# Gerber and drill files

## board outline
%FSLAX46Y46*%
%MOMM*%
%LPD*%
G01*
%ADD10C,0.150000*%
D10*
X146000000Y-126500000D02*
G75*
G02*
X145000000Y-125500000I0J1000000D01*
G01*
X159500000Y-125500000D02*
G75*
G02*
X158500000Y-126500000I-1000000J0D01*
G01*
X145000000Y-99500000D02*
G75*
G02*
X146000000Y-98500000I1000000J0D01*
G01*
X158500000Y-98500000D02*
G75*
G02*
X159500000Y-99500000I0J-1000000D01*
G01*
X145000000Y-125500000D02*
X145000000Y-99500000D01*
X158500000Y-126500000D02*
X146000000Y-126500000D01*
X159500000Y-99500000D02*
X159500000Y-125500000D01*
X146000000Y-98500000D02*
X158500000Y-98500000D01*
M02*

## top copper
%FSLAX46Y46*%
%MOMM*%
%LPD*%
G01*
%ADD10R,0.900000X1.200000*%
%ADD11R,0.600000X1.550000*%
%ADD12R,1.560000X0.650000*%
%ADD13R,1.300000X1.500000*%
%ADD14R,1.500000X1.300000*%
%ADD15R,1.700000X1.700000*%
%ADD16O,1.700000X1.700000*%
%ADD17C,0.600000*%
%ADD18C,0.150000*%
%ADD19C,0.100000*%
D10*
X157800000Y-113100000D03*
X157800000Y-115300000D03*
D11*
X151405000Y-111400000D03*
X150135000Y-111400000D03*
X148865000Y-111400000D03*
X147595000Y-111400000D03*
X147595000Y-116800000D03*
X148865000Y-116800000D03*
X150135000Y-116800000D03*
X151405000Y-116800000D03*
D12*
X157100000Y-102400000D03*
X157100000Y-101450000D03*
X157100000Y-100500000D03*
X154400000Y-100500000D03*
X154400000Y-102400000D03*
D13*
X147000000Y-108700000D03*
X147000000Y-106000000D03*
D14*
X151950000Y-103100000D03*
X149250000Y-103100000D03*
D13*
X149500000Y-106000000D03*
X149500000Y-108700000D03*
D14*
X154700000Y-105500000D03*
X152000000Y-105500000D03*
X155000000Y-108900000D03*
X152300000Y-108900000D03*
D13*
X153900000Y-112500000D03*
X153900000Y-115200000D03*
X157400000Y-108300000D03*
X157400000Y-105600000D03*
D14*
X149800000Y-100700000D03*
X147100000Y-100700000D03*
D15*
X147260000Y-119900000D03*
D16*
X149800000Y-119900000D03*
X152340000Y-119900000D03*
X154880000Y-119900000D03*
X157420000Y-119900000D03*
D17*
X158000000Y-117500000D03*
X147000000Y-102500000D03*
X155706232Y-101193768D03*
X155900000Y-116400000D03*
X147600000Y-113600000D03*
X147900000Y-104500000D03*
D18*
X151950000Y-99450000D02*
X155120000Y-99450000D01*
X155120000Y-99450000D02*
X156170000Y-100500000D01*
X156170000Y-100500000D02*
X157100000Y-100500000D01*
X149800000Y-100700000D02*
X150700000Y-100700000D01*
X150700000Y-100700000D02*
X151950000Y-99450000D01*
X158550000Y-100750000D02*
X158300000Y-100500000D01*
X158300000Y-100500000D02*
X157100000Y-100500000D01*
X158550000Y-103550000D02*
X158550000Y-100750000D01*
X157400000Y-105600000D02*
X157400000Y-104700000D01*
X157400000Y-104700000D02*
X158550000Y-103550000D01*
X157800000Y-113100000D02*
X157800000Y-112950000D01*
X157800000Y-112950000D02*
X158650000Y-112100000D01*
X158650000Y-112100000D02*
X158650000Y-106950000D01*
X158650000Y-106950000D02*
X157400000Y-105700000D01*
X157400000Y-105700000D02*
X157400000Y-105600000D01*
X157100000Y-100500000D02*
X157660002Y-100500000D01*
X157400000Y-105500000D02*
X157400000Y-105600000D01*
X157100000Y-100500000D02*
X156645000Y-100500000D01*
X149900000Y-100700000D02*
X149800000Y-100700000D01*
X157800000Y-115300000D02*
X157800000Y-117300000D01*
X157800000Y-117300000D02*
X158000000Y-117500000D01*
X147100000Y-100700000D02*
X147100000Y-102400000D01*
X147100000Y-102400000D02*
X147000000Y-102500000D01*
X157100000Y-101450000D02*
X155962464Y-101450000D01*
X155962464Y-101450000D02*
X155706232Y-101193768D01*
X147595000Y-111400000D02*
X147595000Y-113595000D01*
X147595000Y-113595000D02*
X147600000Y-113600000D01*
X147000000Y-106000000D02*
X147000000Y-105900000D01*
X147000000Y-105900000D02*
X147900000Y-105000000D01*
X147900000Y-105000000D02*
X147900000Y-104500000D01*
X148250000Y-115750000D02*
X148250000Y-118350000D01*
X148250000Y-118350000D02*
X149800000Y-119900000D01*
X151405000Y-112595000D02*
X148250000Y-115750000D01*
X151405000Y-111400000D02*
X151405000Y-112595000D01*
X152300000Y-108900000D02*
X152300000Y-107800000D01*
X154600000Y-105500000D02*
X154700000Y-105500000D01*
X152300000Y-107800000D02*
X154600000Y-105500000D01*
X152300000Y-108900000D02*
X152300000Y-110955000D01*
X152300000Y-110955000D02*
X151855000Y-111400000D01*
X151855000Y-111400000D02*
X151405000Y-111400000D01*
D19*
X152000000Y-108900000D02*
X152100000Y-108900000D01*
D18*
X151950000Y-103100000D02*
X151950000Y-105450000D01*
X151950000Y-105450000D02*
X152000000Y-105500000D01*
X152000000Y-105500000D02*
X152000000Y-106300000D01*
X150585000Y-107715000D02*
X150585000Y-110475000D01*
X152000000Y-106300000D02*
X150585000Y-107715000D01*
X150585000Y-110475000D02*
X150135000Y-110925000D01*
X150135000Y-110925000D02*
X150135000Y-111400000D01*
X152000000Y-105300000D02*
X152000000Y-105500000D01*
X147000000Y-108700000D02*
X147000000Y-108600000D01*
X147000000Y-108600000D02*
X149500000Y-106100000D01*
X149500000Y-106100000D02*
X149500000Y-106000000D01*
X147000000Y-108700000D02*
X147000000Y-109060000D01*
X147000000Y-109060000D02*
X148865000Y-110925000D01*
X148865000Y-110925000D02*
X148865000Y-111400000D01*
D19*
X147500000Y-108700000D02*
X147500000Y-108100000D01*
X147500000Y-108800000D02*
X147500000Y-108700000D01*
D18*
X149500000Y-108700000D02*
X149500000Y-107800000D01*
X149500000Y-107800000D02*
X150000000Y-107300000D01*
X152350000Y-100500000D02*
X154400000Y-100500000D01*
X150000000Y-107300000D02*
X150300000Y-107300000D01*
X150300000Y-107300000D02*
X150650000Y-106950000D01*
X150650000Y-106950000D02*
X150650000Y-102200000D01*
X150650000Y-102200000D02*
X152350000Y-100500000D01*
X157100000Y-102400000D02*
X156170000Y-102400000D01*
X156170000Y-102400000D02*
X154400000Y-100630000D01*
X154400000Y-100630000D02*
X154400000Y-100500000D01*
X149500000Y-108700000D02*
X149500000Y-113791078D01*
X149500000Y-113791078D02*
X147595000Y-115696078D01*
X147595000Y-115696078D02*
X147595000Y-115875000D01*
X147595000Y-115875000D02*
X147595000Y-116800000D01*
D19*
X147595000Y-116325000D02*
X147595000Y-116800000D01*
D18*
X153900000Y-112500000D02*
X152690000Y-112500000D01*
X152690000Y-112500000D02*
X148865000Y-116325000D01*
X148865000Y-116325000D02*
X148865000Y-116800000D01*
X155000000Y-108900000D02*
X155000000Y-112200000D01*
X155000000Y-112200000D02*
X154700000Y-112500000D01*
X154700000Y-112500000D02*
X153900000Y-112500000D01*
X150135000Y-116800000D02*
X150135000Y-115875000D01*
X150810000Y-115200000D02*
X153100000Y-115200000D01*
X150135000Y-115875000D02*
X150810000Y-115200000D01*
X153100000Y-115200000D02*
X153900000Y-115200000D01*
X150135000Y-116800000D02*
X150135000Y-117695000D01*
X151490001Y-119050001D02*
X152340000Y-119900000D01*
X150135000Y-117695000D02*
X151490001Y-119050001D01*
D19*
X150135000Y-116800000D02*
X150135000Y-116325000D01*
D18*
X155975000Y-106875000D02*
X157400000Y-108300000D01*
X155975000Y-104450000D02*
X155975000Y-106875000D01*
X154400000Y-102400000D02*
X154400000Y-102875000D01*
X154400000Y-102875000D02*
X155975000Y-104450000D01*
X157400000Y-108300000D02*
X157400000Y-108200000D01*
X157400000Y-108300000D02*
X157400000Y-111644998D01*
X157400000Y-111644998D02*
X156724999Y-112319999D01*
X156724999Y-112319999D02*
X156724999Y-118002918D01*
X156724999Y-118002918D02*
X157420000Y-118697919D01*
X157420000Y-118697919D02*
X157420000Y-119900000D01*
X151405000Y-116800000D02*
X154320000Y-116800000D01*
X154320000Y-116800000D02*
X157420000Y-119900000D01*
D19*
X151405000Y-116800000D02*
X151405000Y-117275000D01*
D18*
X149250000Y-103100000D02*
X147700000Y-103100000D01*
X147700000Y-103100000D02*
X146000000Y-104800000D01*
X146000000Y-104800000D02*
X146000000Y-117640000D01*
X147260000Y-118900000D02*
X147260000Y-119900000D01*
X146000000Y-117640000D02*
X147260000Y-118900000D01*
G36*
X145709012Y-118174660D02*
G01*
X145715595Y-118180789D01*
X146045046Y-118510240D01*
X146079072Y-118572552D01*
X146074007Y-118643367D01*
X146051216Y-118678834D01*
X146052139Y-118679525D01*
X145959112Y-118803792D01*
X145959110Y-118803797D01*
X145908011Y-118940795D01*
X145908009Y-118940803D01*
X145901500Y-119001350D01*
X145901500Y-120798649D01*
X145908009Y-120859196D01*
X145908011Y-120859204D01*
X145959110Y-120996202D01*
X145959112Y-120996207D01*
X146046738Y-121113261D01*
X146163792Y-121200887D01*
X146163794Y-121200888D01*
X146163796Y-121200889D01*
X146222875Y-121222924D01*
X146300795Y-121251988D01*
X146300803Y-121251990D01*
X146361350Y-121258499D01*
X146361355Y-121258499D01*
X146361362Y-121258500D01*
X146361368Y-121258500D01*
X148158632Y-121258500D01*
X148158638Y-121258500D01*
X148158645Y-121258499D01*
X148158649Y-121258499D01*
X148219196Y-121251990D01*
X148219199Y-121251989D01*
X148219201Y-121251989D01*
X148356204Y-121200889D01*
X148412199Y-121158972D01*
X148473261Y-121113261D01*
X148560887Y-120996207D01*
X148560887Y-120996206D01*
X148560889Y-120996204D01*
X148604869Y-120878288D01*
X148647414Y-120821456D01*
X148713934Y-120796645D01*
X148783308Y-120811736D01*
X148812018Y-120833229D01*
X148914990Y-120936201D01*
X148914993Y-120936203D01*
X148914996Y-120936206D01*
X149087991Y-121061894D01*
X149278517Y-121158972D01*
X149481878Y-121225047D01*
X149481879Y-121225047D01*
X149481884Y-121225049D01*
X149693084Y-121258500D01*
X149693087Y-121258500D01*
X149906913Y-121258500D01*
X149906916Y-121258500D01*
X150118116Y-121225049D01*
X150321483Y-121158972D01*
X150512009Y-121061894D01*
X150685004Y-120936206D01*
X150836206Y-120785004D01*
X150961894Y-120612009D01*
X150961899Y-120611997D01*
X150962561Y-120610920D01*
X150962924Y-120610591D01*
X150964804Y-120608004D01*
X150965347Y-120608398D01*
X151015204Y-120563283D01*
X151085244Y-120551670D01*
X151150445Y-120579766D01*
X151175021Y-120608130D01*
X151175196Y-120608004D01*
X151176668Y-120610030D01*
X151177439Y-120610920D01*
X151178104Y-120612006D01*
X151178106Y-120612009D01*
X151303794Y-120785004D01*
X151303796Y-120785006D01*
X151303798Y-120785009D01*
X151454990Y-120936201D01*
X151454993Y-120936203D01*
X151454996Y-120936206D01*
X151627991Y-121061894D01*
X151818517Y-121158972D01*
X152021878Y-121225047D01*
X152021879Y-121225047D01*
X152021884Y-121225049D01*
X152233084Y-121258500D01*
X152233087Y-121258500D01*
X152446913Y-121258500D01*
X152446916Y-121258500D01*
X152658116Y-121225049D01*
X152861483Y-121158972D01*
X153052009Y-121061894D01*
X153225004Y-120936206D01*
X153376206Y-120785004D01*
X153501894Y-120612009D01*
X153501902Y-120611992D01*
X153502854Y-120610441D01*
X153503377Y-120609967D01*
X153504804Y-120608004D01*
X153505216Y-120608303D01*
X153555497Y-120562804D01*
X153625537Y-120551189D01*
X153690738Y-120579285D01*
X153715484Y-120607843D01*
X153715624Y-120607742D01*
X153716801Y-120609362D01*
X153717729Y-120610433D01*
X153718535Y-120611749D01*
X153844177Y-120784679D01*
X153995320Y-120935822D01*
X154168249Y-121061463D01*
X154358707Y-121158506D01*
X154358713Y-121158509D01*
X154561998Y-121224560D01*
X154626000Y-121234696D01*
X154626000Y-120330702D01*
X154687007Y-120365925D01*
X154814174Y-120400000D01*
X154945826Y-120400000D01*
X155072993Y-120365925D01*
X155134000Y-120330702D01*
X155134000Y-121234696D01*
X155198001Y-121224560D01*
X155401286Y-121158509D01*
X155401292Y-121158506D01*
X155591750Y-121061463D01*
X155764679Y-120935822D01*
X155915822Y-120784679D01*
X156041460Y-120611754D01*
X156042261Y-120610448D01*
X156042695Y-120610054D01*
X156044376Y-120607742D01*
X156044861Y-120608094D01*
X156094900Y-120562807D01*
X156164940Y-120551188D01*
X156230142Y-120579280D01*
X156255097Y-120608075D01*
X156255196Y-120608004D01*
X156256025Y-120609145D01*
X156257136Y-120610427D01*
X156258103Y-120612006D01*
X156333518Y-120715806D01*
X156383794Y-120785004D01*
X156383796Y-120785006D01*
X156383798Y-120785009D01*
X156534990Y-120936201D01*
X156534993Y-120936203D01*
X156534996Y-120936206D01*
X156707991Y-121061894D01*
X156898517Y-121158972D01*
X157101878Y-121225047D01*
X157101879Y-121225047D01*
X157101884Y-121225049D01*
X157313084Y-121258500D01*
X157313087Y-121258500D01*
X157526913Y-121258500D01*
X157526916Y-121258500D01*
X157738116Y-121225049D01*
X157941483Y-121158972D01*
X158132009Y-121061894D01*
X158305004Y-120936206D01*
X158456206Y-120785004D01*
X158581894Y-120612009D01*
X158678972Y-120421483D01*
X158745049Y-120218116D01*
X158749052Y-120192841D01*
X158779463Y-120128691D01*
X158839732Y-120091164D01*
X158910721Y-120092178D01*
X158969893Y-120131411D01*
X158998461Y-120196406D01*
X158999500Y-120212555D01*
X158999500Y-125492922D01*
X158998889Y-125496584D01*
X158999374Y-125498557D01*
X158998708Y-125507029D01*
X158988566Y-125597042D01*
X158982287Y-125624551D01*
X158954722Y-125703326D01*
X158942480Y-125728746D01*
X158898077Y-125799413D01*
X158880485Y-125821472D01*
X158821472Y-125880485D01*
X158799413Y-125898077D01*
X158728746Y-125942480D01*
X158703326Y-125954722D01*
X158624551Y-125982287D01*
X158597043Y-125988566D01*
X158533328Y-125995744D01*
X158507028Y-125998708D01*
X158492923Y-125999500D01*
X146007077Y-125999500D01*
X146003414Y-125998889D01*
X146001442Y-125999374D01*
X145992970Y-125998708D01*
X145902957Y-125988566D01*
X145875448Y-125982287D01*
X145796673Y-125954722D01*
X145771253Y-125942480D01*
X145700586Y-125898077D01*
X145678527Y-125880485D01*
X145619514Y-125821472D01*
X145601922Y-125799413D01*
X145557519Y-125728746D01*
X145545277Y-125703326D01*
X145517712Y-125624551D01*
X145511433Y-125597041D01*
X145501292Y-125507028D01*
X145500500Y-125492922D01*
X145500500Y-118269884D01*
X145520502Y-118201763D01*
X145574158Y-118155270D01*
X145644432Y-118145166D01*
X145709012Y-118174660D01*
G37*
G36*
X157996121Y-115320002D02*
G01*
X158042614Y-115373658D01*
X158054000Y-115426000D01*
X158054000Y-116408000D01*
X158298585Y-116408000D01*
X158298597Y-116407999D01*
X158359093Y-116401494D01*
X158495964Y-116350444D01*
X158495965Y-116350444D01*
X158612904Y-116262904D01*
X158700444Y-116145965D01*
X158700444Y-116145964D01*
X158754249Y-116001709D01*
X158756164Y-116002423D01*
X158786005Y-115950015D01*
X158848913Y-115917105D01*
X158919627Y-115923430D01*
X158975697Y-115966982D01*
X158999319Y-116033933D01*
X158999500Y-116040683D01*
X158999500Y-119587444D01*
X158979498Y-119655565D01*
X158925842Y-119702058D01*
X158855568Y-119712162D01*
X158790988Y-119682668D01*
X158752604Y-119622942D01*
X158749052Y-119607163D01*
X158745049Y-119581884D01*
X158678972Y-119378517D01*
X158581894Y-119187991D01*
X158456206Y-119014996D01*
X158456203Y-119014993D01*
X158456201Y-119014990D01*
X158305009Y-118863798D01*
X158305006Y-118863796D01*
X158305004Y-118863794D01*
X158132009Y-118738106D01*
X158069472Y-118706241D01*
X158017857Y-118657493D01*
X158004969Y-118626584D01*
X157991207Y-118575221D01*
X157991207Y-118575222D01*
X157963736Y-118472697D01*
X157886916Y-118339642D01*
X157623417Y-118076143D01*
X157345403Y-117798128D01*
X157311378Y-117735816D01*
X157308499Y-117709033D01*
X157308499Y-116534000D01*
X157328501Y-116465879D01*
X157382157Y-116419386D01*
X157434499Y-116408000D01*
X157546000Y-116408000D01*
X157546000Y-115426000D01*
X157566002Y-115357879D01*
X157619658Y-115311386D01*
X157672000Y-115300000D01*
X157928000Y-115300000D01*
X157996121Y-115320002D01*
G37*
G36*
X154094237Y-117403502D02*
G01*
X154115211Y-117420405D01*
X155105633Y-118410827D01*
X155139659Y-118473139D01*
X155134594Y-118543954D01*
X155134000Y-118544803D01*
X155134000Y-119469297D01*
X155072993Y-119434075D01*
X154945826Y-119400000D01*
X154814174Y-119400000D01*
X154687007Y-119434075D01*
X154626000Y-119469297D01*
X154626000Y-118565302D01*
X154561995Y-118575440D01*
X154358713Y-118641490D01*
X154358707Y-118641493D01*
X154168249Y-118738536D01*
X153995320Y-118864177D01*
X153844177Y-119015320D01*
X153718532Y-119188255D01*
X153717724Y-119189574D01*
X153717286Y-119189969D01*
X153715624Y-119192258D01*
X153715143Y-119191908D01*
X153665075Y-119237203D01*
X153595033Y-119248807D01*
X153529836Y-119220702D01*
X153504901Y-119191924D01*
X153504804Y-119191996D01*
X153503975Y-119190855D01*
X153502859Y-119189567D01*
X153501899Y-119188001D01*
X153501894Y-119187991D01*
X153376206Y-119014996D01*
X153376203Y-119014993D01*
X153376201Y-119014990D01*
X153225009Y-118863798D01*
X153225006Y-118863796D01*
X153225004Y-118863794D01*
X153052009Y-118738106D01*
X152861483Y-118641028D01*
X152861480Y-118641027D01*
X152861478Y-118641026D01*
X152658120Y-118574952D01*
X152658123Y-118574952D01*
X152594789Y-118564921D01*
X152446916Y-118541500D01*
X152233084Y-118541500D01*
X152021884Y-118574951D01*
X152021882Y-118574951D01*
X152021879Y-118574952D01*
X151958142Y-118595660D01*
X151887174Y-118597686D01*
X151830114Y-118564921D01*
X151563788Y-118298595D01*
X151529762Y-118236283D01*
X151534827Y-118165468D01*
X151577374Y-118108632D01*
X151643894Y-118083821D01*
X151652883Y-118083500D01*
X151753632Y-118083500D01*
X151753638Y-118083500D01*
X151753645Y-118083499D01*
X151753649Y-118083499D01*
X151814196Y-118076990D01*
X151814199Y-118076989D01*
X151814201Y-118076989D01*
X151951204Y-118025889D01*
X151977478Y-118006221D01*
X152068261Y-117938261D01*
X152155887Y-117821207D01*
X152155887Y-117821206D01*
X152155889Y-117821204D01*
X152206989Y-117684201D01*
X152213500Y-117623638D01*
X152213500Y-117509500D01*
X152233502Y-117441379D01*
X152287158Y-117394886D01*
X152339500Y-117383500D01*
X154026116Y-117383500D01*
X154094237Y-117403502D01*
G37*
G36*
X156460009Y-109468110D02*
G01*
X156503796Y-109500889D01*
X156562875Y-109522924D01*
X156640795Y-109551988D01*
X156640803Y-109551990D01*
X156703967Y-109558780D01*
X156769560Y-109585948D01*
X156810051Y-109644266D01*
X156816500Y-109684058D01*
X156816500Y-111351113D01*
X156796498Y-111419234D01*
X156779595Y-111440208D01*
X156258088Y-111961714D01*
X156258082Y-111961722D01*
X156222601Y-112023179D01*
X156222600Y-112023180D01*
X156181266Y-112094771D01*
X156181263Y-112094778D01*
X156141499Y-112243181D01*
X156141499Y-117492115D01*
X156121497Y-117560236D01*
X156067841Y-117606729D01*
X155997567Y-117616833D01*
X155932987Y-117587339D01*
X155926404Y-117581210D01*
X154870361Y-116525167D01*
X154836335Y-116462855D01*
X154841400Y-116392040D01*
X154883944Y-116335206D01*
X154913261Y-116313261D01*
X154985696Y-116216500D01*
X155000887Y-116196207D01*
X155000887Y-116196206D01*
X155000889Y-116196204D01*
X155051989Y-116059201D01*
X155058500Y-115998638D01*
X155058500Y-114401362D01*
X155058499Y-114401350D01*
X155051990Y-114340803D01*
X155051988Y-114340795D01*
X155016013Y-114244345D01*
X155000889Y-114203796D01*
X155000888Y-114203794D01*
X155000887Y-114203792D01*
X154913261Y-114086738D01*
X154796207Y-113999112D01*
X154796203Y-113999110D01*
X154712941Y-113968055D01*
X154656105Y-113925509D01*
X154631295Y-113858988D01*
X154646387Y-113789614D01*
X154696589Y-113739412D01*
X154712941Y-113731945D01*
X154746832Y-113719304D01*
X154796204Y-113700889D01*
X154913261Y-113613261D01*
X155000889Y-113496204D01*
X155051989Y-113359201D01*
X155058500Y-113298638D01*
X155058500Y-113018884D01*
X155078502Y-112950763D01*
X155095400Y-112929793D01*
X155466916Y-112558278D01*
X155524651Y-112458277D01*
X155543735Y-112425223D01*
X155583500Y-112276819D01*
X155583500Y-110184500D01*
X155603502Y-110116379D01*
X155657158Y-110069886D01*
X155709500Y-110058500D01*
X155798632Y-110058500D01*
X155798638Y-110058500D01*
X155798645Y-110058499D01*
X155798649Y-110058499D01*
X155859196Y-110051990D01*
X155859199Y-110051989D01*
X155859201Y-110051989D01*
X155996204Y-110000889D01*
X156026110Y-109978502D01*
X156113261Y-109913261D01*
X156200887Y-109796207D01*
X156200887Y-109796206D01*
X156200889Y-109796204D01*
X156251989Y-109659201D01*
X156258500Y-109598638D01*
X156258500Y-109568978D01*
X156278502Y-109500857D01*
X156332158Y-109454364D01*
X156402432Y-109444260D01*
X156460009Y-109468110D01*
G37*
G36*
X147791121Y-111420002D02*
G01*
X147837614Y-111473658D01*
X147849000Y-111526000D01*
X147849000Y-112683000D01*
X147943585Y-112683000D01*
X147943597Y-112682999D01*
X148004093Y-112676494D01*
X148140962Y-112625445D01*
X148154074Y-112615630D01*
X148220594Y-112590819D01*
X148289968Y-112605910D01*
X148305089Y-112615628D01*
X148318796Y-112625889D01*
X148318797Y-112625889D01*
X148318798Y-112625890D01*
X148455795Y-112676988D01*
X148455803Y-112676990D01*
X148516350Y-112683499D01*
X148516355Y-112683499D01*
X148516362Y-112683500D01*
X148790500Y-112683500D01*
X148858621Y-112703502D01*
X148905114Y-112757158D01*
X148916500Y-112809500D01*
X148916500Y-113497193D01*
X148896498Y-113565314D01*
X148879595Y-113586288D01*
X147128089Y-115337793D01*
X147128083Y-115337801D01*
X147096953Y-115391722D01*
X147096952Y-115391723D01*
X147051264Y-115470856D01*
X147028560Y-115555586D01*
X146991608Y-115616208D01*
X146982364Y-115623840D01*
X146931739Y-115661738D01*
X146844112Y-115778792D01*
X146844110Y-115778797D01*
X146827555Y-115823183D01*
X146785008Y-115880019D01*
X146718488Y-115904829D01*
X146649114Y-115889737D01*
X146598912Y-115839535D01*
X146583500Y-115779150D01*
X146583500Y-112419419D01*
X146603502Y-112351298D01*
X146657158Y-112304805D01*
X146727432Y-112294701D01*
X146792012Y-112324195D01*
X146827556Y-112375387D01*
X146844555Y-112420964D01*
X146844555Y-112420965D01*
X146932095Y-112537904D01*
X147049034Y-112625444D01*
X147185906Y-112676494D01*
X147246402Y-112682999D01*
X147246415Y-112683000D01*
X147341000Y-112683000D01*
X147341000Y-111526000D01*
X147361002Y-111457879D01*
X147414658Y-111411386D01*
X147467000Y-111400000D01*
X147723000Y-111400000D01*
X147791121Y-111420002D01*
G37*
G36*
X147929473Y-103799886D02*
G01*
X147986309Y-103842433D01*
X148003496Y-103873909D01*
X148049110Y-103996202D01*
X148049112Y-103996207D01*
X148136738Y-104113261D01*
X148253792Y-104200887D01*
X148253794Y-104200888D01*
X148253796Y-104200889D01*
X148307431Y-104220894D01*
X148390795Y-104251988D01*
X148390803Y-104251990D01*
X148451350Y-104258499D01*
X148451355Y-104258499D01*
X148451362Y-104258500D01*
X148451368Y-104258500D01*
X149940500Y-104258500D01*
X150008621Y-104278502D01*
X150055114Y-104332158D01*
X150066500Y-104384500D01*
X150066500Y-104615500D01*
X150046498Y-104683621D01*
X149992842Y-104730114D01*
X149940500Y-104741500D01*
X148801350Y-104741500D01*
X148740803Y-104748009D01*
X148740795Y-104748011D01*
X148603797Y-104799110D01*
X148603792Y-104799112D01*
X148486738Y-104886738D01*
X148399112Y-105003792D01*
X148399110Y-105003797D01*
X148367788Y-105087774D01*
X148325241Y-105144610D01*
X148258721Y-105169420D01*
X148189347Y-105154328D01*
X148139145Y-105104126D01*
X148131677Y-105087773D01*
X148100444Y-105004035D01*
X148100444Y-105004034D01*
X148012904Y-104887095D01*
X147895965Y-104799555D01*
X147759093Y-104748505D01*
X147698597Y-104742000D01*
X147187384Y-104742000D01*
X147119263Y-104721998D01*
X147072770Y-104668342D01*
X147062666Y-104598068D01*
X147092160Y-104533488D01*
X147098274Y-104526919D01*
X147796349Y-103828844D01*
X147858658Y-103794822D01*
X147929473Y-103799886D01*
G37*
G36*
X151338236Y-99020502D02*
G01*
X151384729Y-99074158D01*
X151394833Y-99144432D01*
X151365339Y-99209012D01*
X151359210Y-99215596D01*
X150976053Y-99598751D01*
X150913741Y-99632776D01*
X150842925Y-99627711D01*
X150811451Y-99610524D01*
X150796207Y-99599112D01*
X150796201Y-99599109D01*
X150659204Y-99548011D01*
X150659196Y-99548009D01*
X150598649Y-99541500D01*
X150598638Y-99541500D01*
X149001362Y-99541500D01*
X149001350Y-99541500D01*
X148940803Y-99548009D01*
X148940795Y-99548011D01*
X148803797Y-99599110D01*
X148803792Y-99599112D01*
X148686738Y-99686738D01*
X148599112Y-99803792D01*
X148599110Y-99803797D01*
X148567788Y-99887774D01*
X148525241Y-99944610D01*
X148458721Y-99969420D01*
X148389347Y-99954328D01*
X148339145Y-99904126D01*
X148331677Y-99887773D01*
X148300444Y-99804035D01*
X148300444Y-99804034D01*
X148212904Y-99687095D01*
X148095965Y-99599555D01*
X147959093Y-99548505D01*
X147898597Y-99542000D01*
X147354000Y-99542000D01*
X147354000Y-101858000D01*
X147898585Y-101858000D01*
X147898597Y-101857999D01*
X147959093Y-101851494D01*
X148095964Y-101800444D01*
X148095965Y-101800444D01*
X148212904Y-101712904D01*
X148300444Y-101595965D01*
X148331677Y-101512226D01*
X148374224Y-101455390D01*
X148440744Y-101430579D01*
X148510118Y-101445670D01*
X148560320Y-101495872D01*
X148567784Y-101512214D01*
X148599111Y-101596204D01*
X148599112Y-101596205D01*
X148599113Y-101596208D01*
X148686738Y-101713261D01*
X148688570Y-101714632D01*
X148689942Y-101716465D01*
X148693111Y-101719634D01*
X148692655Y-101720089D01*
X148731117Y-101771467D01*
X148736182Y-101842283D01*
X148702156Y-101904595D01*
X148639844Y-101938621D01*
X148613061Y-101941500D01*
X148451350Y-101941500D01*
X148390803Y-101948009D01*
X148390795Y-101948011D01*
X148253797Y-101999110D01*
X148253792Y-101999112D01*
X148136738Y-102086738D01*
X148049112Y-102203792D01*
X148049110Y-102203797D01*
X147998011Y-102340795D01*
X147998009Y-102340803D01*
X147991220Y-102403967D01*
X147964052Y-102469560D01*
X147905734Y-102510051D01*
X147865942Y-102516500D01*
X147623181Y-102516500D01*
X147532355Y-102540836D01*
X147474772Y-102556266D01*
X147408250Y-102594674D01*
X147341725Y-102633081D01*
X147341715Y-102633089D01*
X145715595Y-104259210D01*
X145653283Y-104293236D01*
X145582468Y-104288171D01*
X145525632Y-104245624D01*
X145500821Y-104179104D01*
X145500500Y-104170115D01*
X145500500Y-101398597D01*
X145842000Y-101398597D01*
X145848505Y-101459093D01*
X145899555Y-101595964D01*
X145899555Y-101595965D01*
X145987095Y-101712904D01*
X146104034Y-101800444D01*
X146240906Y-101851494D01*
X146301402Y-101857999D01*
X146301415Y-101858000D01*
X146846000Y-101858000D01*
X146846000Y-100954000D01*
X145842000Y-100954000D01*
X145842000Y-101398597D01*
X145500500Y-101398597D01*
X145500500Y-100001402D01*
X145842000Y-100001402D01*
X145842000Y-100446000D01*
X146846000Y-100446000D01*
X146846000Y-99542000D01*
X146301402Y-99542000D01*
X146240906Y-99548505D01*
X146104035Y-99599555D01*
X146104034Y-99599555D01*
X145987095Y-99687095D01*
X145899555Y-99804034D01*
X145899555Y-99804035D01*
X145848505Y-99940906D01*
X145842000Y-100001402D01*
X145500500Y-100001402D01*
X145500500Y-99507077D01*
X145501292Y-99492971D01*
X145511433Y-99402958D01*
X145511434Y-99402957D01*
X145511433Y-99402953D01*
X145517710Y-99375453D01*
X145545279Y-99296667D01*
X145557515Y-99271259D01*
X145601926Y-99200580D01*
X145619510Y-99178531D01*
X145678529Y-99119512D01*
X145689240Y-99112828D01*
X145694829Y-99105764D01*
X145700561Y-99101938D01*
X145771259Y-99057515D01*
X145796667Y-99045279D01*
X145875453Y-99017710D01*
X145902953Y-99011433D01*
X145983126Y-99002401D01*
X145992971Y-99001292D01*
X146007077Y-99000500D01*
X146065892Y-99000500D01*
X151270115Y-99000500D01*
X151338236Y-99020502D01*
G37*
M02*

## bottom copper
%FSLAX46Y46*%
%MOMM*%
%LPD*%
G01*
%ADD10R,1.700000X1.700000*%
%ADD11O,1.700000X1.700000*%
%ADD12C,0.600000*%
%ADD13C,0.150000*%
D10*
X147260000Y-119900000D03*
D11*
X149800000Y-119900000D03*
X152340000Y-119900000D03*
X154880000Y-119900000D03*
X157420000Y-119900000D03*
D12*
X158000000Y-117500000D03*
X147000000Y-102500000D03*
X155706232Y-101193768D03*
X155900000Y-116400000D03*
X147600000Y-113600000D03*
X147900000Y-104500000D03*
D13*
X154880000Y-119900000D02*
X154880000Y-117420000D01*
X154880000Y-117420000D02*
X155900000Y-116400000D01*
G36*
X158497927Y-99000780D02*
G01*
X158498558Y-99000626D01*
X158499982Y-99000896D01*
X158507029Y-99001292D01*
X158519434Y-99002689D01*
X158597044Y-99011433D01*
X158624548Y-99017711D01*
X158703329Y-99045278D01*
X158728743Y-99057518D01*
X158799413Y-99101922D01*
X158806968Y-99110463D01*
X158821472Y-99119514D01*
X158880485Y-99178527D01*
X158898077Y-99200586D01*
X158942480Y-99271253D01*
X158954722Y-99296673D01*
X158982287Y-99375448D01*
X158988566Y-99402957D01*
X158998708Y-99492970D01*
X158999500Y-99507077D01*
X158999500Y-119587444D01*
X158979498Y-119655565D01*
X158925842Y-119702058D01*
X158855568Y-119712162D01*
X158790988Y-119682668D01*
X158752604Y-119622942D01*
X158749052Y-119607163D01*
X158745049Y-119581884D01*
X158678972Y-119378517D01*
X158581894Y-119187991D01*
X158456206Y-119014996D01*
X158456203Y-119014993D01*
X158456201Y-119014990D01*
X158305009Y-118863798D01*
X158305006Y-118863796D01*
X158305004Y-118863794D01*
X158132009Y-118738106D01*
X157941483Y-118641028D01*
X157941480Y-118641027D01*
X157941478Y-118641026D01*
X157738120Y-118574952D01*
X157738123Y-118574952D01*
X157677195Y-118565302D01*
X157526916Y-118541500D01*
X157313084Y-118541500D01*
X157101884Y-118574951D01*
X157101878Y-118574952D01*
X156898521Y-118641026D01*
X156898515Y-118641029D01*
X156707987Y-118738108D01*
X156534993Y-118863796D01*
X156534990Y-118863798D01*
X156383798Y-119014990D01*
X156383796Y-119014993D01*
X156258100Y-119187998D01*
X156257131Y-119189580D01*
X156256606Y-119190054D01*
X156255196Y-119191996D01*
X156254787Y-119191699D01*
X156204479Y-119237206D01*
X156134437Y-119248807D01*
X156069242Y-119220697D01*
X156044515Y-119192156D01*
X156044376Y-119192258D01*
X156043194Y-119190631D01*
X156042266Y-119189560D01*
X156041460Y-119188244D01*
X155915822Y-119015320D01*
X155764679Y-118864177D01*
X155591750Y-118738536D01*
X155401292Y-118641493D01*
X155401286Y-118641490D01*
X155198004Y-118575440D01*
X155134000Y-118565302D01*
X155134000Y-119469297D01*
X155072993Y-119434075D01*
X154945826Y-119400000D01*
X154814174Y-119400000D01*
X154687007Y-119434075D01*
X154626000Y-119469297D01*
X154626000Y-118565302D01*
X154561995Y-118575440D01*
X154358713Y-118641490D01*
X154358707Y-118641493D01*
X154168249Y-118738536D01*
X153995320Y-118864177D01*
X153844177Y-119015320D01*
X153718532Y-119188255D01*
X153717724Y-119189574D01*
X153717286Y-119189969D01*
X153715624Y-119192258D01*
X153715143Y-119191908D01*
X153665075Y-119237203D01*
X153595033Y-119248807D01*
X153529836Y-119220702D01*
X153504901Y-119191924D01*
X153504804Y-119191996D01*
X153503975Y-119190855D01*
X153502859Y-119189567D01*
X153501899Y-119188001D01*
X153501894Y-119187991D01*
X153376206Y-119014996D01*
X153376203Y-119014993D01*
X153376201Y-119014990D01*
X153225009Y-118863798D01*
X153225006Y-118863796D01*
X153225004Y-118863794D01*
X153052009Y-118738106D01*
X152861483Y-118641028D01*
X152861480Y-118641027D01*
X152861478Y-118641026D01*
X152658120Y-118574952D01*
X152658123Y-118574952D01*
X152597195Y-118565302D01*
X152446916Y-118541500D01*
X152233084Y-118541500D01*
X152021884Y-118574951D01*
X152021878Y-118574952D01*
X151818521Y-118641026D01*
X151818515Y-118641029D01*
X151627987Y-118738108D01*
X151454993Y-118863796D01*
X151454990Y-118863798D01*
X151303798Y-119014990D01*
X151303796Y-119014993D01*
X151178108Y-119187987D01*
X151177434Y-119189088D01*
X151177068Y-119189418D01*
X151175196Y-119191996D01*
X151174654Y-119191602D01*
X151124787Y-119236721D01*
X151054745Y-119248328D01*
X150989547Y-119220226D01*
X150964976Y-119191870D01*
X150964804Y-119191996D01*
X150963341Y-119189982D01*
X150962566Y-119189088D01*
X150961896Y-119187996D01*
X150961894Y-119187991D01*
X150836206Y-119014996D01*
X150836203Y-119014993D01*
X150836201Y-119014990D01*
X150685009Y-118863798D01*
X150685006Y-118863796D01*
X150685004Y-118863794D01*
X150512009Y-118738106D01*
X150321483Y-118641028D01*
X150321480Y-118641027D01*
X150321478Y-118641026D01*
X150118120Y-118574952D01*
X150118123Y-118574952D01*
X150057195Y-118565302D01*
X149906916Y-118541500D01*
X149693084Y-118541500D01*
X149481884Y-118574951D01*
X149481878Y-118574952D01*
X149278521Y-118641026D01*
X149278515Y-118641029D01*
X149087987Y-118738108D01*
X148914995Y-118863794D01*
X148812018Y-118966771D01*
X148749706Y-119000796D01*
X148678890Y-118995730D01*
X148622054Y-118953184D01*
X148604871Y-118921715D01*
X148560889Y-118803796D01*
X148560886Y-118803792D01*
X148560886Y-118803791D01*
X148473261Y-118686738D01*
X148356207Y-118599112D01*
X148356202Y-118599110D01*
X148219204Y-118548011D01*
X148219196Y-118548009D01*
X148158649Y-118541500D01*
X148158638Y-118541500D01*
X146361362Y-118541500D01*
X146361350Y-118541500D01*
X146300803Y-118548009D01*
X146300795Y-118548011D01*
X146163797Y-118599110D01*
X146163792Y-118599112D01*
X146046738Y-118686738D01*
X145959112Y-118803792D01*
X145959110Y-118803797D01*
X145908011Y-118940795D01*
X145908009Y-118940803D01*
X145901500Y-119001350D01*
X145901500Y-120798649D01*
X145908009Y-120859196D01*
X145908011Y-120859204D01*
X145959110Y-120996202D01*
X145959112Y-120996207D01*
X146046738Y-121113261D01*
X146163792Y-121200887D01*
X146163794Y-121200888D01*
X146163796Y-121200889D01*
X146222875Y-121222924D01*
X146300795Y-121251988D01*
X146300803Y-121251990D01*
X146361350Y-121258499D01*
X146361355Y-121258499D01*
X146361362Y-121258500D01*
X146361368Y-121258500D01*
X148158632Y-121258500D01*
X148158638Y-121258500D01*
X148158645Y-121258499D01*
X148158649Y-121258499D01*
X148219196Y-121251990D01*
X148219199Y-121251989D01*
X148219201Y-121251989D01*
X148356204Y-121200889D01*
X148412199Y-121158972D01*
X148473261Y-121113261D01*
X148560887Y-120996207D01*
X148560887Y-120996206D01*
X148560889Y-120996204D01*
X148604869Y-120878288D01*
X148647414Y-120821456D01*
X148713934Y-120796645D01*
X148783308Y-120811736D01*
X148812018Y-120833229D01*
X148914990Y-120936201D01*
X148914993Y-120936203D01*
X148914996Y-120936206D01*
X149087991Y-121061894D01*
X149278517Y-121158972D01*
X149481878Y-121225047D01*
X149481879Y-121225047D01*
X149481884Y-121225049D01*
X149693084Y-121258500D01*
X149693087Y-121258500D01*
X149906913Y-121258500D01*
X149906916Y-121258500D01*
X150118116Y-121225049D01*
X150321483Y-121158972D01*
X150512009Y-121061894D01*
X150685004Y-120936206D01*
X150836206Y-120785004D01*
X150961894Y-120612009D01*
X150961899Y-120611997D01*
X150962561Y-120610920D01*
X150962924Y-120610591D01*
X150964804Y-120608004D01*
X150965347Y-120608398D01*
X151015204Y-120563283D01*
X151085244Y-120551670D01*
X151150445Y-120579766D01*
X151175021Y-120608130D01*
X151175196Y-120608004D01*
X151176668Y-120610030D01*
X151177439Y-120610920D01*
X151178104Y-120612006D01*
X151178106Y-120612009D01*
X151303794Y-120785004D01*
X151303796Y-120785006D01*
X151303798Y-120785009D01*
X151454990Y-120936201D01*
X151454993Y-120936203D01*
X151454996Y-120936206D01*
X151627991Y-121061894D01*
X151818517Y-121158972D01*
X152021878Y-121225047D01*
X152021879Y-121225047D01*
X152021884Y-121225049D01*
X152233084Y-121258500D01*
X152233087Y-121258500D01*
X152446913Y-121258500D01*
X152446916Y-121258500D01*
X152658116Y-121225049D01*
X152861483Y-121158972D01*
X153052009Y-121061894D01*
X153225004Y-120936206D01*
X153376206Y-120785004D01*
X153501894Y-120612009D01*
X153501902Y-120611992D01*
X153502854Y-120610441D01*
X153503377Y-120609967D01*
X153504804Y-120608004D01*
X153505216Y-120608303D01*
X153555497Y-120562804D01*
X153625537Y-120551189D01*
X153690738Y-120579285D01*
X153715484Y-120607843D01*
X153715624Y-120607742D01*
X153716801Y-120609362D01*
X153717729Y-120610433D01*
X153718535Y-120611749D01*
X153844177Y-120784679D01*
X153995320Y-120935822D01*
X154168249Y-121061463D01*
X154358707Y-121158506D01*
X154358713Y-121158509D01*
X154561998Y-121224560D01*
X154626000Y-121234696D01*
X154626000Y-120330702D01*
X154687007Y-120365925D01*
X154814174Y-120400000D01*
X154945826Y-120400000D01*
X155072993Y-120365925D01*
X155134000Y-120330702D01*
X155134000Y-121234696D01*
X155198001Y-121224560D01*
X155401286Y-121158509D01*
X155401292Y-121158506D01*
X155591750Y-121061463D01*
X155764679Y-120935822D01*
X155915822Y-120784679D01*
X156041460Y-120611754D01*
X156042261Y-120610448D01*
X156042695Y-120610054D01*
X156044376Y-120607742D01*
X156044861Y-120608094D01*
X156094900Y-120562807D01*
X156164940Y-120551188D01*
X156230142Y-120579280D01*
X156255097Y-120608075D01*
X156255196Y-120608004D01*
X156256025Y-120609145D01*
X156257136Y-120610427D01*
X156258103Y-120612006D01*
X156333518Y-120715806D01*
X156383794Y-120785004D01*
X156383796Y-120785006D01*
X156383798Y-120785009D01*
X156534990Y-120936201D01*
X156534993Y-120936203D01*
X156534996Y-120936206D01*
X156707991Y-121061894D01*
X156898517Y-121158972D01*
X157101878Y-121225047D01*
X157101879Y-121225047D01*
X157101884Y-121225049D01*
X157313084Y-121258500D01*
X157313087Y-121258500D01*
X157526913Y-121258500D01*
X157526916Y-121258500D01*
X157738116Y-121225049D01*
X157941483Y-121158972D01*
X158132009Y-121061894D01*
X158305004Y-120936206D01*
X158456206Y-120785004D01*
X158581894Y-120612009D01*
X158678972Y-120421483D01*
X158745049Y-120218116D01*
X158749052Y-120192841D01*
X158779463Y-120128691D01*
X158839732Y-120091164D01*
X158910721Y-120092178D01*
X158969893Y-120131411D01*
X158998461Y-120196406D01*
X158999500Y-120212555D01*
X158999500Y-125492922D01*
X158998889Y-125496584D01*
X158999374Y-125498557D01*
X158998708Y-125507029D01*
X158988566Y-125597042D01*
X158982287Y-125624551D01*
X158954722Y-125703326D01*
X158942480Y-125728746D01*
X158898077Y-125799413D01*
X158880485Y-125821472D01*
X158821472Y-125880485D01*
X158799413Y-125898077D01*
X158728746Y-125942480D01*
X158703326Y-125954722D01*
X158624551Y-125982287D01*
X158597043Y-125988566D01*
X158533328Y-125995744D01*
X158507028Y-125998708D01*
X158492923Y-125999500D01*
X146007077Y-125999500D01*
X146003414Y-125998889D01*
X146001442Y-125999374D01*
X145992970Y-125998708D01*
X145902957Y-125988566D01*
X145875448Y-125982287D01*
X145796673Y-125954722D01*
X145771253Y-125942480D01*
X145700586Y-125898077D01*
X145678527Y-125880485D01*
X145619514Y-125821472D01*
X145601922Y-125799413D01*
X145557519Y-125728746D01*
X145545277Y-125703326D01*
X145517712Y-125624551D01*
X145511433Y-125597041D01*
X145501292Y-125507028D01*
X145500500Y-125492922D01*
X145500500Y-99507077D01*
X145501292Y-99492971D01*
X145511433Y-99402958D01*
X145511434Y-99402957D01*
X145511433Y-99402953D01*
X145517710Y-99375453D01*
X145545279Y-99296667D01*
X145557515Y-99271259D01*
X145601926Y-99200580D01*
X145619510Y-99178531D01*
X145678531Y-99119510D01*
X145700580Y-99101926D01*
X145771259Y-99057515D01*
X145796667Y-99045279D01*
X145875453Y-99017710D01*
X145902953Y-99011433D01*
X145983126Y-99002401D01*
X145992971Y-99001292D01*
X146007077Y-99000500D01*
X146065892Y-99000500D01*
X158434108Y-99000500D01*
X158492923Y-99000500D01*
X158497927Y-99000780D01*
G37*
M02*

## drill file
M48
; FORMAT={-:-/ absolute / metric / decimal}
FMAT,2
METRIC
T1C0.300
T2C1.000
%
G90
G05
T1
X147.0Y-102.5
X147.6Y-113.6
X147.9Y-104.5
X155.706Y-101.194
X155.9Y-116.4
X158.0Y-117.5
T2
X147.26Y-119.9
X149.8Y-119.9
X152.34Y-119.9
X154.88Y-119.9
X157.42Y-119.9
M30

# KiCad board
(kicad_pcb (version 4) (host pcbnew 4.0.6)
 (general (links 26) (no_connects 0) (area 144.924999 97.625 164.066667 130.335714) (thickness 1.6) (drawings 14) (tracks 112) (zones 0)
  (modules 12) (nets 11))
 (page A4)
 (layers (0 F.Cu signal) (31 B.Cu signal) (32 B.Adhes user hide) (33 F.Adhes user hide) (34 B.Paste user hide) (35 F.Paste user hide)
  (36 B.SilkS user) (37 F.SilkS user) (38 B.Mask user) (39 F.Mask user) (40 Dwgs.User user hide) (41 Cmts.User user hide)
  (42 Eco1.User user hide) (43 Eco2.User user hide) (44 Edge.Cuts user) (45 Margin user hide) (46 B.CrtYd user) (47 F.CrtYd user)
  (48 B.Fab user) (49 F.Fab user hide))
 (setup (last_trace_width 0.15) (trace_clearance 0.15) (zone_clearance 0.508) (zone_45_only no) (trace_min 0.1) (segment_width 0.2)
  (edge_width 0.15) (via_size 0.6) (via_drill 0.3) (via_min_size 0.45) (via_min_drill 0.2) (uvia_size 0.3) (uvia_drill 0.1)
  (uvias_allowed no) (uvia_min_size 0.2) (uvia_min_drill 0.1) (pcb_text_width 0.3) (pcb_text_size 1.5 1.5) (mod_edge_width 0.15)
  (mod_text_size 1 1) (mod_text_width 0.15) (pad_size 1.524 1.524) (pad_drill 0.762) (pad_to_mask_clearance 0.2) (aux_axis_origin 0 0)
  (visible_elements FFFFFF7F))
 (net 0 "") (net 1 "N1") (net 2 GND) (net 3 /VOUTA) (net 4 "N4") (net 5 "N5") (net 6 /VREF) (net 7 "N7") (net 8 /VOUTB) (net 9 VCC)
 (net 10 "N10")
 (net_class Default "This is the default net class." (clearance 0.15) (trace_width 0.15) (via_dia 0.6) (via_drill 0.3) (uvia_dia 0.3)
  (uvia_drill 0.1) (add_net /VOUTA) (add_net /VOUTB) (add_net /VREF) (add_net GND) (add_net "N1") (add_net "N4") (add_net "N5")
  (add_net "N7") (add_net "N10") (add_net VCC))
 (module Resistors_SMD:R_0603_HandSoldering (layer F.Cu) (at 157.8 114.2 270)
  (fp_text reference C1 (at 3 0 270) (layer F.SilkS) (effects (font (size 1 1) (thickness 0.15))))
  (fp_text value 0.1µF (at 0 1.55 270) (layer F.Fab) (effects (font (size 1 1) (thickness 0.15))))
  (pad 1 smd rect (at -1.1 0 270) (size 1.2 0.9) (layers F.Cu F.Paste F.Mask) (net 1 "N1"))
  (pad 2 smd rect (at 1.1 0 270) (size 1.2 0.9) (layers F.Cu F.Paste F.Mask) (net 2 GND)))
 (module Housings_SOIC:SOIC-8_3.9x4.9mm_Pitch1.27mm (layer F.Cu) (at 149.5 114.1 270)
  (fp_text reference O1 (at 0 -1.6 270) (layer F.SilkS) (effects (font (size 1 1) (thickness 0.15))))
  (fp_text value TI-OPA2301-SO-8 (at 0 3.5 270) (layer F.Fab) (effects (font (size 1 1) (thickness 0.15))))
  (pad 1 smd rect (at -2.7 -1.905 270) (size 1.55 0.6) (layers F.Cu F.Paste F.Mask) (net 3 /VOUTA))
  (pad 2 smd rect (at -2.7 -0.635 270) (size 1.55 0.6) (layers F.Cu F.Paste F.Mask) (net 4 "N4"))
  (pad 3 smd rect (at -2.7 0.635 270) (size 1.55 0.6) (layers F.Cu F.Paste F.Mask) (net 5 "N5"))
  (pad 4 smd rect (at -2.7 1.905 270) (size 1.55 0.6) (layers F.Cu F.Paste F.Mask) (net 2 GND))
  (pad 5 smd rect (at 2.7 1.905 270) (size 1.55 0.6) (layers F.Cu F.Paste F.Mask) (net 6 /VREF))
  (pad 6 smd rect (at 2.7 0.635 270) (size 1.55 0.6) (layers F.Cu F.Paste F.Mask) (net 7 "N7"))
  (pad 7 smd rect (at 2.7 -0.635 270) (size 1.55 0.6) (layers F.Cu F.Paste F.Mask) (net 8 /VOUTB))
  (pad 8 smd rect (at 2.7 -1.905 270) (size 1.55 0.6) (layers F.Cu F.Paste F.Mask) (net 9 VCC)))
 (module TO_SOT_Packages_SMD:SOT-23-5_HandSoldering (layer F.Cu) (at 155.75 101.45 180)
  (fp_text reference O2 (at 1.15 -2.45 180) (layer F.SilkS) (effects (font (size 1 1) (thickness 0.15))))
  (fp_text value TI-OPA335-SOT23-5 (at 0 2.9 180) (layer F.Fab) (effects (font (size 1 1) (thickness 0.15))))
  (pad 1 smd rect (at -1.35 -0.95 180) (size 1.56 0.65) (layers F.Cu F.Paste F.Mask) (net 6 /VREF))
  (pad 2 smd rect (at -1.35 0 180) (size 1.56 0.65) (layers F.Cu F.Paste F.Mask) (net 2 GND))
  (pad 3 smd rect (at -1.35 0.95 180) (size 1.56 0.65) (layers F.Cu F.Paste F.Mask) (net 1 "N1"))
  (pad 4 smd rect (at 1.35 0.95 180) (size 1.56 0.65) (layers F.Cu F.Paste F.Mask) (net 6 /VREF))
  (pad 5 smd rect (at 1.35 -0.95 180) (size 1.56 0.65) (layers F.Cu F.Paste F.Mask) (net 9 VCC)))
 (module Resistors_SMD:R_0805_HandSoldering (layer F.Cu) (at 147 107.35 90)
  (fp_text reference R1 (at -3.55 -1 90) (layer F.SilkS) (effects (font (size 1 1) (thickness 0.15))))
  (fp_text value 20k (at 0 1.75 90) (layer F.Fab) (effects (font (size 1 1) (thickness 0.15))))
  (pad 1 smd rect (at -1.35 0 90) (size 1.5 1.3) (layers F.Cu F.Paste F.Mask) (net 5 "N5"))
  (pad 2 smd rect (at 1.35 0 90) (size 1.5 1.3) (layers F.Cu F.Paste F.Mask) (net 2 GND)))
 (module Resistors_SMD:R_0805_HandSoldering (layer F.Cu) (at 150.6 103.1 180)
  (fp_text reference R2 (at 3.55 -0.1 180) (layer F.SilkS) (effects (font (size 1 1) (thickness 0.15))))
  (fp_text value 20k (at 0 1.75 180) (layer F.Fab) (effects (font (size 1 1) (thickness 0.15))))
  (pad 1 smd rect (at -1.35 0 180) (size 1.5 1.3) (layers F.Cu F.Paste F.Mask) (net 4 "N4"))
  (pad 2 smd rect (at 1.35 0 180) (size 1.5 1.3) (layers F.Cu F.Paste F.Mask) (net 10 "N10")))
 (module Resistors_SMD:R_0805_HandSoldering (layer F.Cu) (at 149.5 107.35 270)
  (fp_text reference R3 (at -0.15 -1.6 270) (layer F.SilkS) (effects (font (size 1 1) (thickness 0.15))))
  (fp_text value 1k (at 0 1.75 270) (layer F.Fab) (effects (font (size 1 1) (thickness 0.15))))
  (pad 1 smd rect (at -1.35 0 270) (size 1.5 1.3) (layers F.Cu F.Paste F.Mask) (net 5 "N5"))
  (pad 2 smd rect (at 1.35 0 270) (size 1.5 1.3) (layers F.Cu F.Paste F.Mask) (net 6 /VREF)))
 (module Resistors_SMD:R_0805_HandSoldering (layer F.Cu) (at 153.35 105.5 180)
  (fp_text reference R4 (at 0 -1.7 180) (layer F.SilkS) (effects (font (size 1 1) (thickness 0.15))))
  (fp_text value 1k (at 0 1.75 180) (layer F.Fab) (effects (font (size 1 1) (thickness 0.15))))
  (pad 1 smd rect (at -1.35 0 180) (size 1.5 1.3) (layers F.Cu F.Paste F.Mask) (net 3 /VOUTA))
  (pad 2 smd rect (at 1.35 0 180) (size 1.5 1.3) (layers F.Cu F.Paste F.Mask) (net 4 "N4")))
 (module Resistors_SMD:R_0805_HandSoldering (layer F.Cu) (at 153.65 108.9 180)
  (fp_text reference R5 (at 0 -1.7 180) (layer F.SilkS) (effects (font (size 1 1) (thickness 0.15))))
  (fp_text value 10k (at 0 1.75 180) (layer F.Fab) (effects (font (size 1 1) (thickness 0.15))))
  (pad 1 smd rect (at -1.35 0 180) (size 1.5 1.3) (layers F.Cu F.Paste F.Mask) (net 7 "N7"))
  (pad 2 smd rect (at 1.35 0 180) (size 1.5 1.3) (layers F.Cu F.Paste F.Mask) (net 3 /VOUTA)))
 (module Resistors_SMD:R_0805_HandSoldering (layer F.Cu) (at 153.9 113.85 270)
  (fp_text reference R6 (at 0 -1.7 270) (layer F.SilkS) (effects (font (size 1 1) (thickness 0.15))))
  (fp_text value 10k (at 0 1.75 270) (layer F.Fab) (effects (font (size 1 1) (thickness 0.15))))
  (pad 1 smd rect (at -1.35 0 270) (size 1.5 1.3) (layers F.Cu F.Paste F.Mask) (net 7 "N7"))
  (pad 2 smd rect (at 1.35 0 270) (size 1.5 1.3) (layers F.Cu F.Paste F.Mask) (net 8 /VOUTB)))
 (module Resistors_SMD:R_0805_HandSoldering (layer F.Cu) (at 157.4 106.95 90)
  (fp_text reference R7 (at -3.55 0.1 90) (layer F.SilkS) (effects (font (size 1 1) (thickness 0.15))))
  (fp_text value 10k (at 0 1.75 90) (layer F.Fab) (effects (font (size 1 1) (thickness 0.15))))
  (pad 1 smd rect (at -1.35 0 90) (size 1.5 1.3) (layers F.Cu F.Paste F.Mask) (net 9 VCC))
  (pad 2 smd rect (at 1.35 0 90) (size 1.5 1.3) (layers F.Cu F.Paste F.Mask) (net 1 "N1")))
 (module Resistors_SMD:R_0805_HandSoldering (layer F.Cu) (at 148.45 100.7 180)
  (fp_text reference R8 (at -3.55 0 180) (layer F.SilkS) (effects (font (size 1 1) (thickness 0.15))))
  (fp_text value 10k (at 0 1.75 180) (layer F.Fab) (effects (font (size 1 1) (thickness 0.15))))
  (pad 1 smd rect (at -1.35 0 180) (size 1.5 1.3) (layers F.Cu F.Paste F.Mask) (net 1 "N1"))
  (pad 2 smd rect (at 1.35 0 180) (size 1.5 1.3) (layers F.Cu F.Paste F.Mask) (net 2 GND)))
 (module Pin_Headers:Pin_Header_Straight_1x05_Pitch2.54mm (layer F.Cu) (at 147.26 119.9 90)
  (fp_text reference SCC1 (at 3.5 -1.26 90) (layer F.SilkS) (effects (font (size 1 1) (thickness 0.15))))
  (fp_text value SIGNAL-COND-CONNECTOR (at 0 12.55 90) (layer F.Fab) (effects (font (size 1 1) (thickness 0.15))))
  (pad 1 thru_hole rect (at 0 0 90) (size 1.7 1.7) (drill 1) (layers *.Cu *.Mask) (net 10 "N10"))
  (pad 2 thru_hole oval (at 0 2.54 90) (size 1.7 1.7) (drill 1) (layers *.Cu *.Mask) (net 3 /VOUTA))
  (pad 3 thru_hole oval (at 0 5.08 90) (size 1.7 1.7) (drill 1) (layers *.Cu *.Mask) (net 8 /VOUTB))
  (pad 4 thru_hole oval (at 0 7.62 90) (size 1.7 1.7) (drill 1) (layers *.Cu *.Mask) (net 2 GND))
  (pad 5 thru_hole oval (at 0 10.16 90) (size 1.7 1.7) (drill 1) (layers *.Cu *.Mask) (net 9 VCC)))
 (gr_arc (start 146 125.5) (end 146 126.5) (angle 90) (layer Edge.Cuts) (width 0.15))
 (gr_arc (start 158.5 125.5) (end 159.5 125.5) (angle 90) (layer Edge.Cuts) (width 0.15))
 (gr_arc (start 146 99.5) (end 145 99.5) (angle 90) (layer Edge.Cuts) (width 0.15))
 (gr_arc (start 158.5 99.5) (end 158.5 98.5) (angle 90) (layer Edge.Cuts) (width 0.15))
 (gr_line (start 145 125.5) (end 145 99.5) (layer Edge.Cuts) (width 0.15))
 (gr_line (start 158.5 126.5) (end 146 126.5) (layer Edge.Cuts) (width 0.15))
 (gr_line (start 159.5 99.5) (end 159.5 125.5) (layer Edge.Cuts) (width 0.15))
 (gr_line (start 146 98.5) (end 158.5 98.5) (layer Edge.Cuts) (width 0.15))
 (segment (start 151.95 99.45) (end 155.12 99.45) (width 0.15) (layer F.Cu) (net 1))
 (segment (start 155.12 99.45) (end 156.17 100.5) (width 0.15) (layer F.Cu) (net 1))
 (segment (start 156.17 100.5) (end 157.1 100.5) (width 0.15) (layer F.Cu) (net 1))
 (segment (start 149.8 100.7) (end 150.7 100.7) (width 0.15) (layer F.Cu) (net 1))
 (segment (start 150.7 100.7) (end 151.95 99.45) (width 0.15) (layer F.Cu) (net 1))
 (segment (start 158.55 100.75) (end 158.3 100.5) (width 0.15) (layer F.Cu) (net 1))
 (segment (start 158.3 100.5) (end 157.1 100.5) (width 0.15) (layer F.Cu) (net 1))
 (segment (start 158.55 103.55) (end 158.55 100.75) (width 0.15) (layer F.Cu) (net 1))
 (segment (start 157.4 105.6) (end 157.4 104.7) (width 0.15) (layer F.Cu) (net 1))
 (segment (start 157.4 104.7) (end 158.55 103.55) (width 0.15) (layer F.Cu) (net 1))
 (segment (start 157.8 113.1) (end 157.8 112.95) (width 0.15) (layer F.Cu) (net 1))
 (segment (start 157.8 112.95) (end 158.65 112.1) (width 0.15) (layer F.Cu) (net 1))
 (segment (start 158.65 112.1) (end 158.65 106.95) (width 0.15) (layer F.Cu) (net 1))
 (segment (start 158.65 106.95) (end 157.4 105.7) (width 0.15) (layer F.Cu) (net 1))
 (segment (start 157.4 105.7) (end 157.4 105.6) (width 0.15) (layer F.Cu) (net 1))
 (segment (start 157.1 100.5) (end 157.660002 100.5) (width 0.15) (layer F.Cu) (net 1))
 (segment (start 157.4 105.5) (end 157.4 105.6) (width 0.15) (layer F.Cu) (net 1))
 (segment (start 157.1 100.5) (end 156.645 100.5) (width 0.15) (layer F.Cu) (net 1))
 (segment (start 149.9 100.7) (end 149.8 100.7) (width 0.15) (layer F.Cu) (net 1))
 (segment (start 157.8 115.3) (end 157.8 117.3) (width 0.15) (layer F.Cu) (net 2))
 (segment (start 157.8 117.3) (end 158 117.5) (width 0.15) (layer F.Cu) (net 2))
 (via (at 158 117.5) (size 0.6) (drill 0.3) (layers F.Cu B.Cu) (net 2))
 (segment (start 147.1 100.7) (end 147.1 102.4) (width 0.15) (layer F.Cu) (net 2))
 (via (at 147 102.5) (size 0.6) (drill 0.3) (layers F.Cu B.Cu) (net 2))
 (segment (start 147.1 102.4) (end 147 102.5) (width 0.15) (layer F.Cu) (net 2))
 (segment (start 157.1 101.45) (end 155.962464 101.45) (width 0.15) (layer F.Cu) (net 2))
 (segment (start 155.962464 101.45) (end 155.706232 101.193768) (width 0.15) (layer F.Cu) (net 2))
 (via (at 155.706232 101.193768) (size 0.6) (drill 0.3) (layers F.Cu B.Cu) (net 2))
 (segment (start 154.88 119.9) (end 154.88 117.42) (width 0.15) (layer B.Cu) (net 2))
 (segment (start 154.88 117.42) (end 155.9 116.4) (width 0.15) (layer B.Cu) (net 2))
 (via (at 155.9 116.4) (size 0.6) (drill 0.3) (layers F.Cu B.Cu) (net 2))
 (segment (start 147.595 111.4) (end 147.595 113.595) (width 0.15) (layer F.Cu) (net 2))
 (segment (start 147.595 113.595) (end 147.6 113.6) (width 0.15) (layer F.Cu) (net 2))
 (via (at 147.6 113.6) (size 0.6) (drill 0.3) (layers F.Cu B.Cu) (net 2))
 (segment (start 147 106) (end 147 105.9) (width 0.15) (layer F.Cu) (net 2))
 (segment (start 147 105.9) (end 147.9 105) (width 0.15) (layer F.Cu) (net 2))
 (segment (start 147.9 105) (end 147.9 104.5) (width 0.15) (layer F.Cu) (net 2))
 (via (at 147.9 104.5) (size 0.6) (drill 0.3) (layers F.Cu B.Cu) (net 2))
 (segment (start 148.25 115.75) (end 148.25 118.35) (width 0.15) (layer F.Cu) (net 3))
 (segment (start 148.25 118.35) (end 149.8 119.9) (width 0.15) (layer F.Cu) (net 3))
 (segment (start 151.405 112.595) (end 148.25 115.75) (width 0.15) (layer F.Cu) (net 3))
 (segment (start 151.405 111.4) (end 151.405 112.595) (width 0.15) (layer F.Cu) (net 3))
 (segment (start 152.3 108.9) (end 152.3 107.8) (width 0.15) (layer F.Cu) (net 3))
 (segment (start 154.6 105.5) (end 154.7 105.5) (width 0.15) (layer F.Cu) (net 3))
 (segment (start 152.3 107.8) (end 154.6 105.5) (width 0.15) (layer F.Cu) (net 3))
 (segment (start 152.3 108.9) (end 152.3 110.955) (width 0.15) (layer F.Cu) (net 3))
 (segment (start 152.3 110.955) (end 151.855 111.4) (width 0.15) (layer F.Cu) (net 3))
 (segment (start 151.855 111.4) (end 151.405 111.4) (width 0.15) (layer F.Cu) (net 3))
 (segment (start 152 108.9) (end 152.1 108.9) (width 0.1) (layer F.Cu) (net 3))
 (segment (start 151.95 103.1) (end 151.95 105.45) (width 0.15) (layer F.Cu) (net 4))
 (segment (start 151.95 105.45) (end 152 105.5) (width 0.15) (layer F.Cu) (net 4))
 (segment (start 152 105.5) (end 152 106.3) (width 0.15) (layer F.Cu) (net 4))
 (segment (start 150.585 107.715) (end 150.585 110.475) (width 0.15) (layer F.Cu) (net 4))
 (segment (start 152 106.3) (end 150.585 107.715) (width 0.15) (layer F.Cu) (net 4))
 (segment (start 150.585 110.475) (end 150.135 110.925) (width 0.15) (layer F.Cu) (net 4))
 (segment (start 150.135 110.925) (end 150.135 111.4) (width 0.15) (layer F.Cu) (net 4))
 (segment (start 152 105.3) (end 152 105.5) (width 0.15) (layer F.Cu) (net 4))
 (segment (start 147 108.7) (end 147 108.6) (width 0.15) (layer F.Cu) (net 5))
 (segment (start 147 108.6) (end 149.5 106.1) (width 0.15) (layer F.Cu) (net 5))
 (segment (start 149.5 106.1) (end 149.5 106) (width 0.15) (layer F.Cu) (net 5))
 (segment (start 147 108.7) (end 147 109.06) (width 0.15) (layer F.Cu) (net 5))
 (segment (start 147 109.06) (end 148.865 110.925) (width 0.15) (layer F.Cu) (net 5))
 (segment (start 148.865 110.925) (end 148.865 111.4) (width 0.15) (layer F.Cu) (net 5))
 (segment (start 147.5 108.7) (end 147.5 108.1) (width 0.1) (layer F.Cu) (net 5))
 (segment (start 147.5 108.8) (end 147.5 108.7) (width 0.1) (layer F.Cu) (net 5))
 (segment (start 149.5 108.7) (end 149.5 107.8) (width 0.15) (layer F.Cu) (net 6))
 (segment (start 149.5 107.8) (end 150 107.3) (width 0.15) (layer F.Cu) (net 6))
 (segment (start 152.35 100.5) (end 154.4 100.5) (width 0.15) (layer F.Cu) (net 6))
 (segment (start 150 107.3) (end 150.3 107.3) (width 0.15) (layer F.Cu) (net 6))
 (segment (start 150.3 107.3) (end 150.65 106.95) (width 0.15) (layer F.Cu) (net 6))
 (segment (start 150.65 106.95) (end 150.65 102.2) (width 0.15) (layer F.Cu) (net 6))
 (segment (start 150.65 102.2) (end 152.35 100.5) (width 0.15) (layer F.Cu) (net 6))
 (segment (start 157.1 102.4) (end 156.17 102.4) (width 0.15) (layer F.Cu) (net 6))
 (segment (start 156.17 102.4) (end 154.4 100.63) (width 0.15) (layer F.Cu) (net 6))
 (segment (start 154.4 100.63) (end 154.4 100.5) (width 0.15) (layer F.Cu) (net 6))
 (segment (start 149.5 108.7) (end 149.5 113.791078) (width 0.15) (layer F.Cu) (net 6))
 (segment (start 149.5 113.791078) (end 147.595 115.696078) (width 0.15) (layer F.Cu) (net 6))
 (segment (start 147.595 115.696078) (end 147.595 115.875) (width 0.15) (layer F.Cu) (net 6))
 (segment (start 147.595 115.875) (end 147.595 116.8) (width 0.15) (layer F.Cu) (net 6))
 (segment (start 147.595 116.325) (end 147.595 116.8) (width 0.1) (layer F.Cu) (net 6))
 (segment (start 153.9 112.5) (end 152.69 112.5) (width 0.15) (layer F.Cu) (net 7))
 (segment (start 152.69 112.5) (end 148.865 116.325) (width 0.15) (layer F.Cu) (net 7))
 (segment (start 148.865 116.325) (end 148.865 116.8) (width 0.15) (layer F.Cu) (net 7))
 (segment (start 155 108.9) (end 155 112.2) (width 0.15) (layer F.Cu) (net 7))
 (segment (start 155 112.2) (end 154.7 112.5) (width 0.15) (layer F.Cu) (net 7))
 (segment (start 154.7 112.5) (end 153.9 112.5) (width 0.15) (layer F.Cu) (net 7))
 (segment (start 150.135 116.8) (end 150.135 115.875) (width 0.15) (layer F.Cu) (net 8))
 (segment (start 150.81 115.2) (end 153.1 115.2) (width 0.15) (layer F.Cu) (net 8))
 (segment (start 150.135 115.875) (end 150.81 115.2) (width 0.15) (layer F.Cu) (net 8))
 (segment (start 153.1 115.2) (end 153.9 115.2) (width 0.15) (layer F.Cu) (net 8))
 (segment (start 150.135 116.8) (end 150.135 117.695) (width 0.15) (layer F.Cu) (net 8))
 (segment (start 151.490001 119.050001) (end 152.34 119.9) (width 0.15) (layer F.Cu) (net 8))
 (segment (start 150.135 117.695) (end 151.490001 119.050001) (width 0.15) (layer F.Cu) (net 8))
 (segment (start 150.135 116.8) (end 150.135 116.325) (width 0.1) (layer F.Cu) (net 8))
 (segment (start 155.975 106.875) (end 157.4 108.3) (width 0.15) (layer F.Cu) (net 9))
 (segment (start 155.975 104.45) (end 155.975 106.875) (width 0.15) (layer F.Cu) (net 9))
 (segment (start 154.4 102.4) (end 154.4 102.875) (width 0.15) (layer F.Cu) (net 9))
 (segment (start 154.4 102.875) (end 155.975 104.45) (width 0.15) (layer F.Cu) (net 9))
 (segment (start 157.4 108.3) (end 157.4 108.2) (width 0.15) (layer F.Cu) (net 9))
 (segment (start 157.4 108.3) (end 157.4 111.644998) (width 0.15) (layer F.Cu) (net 9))
 (segment (start 157.4 111.644998) (end 156.724999 112.319999) (width 0.15) (layer F.Cu) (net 9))
 (segment (start 156.724999 112.319999) (end 156.724999 118.002918) (width 0.15) (layer F.Cu) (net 9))
 (segment (start 156.724999 118.002918) (end 157.42 118.697919) (width 0.15) (layer F.Cu) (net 9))
 (segment (start 157.42 118.697919) (end 157.42 119.9) (width 0.15) (layer F.Cu) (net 9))
 (segment (start 151.405 116.8) (end 154.32 116.8) (width 0.15) (layer F.Cu) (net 9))
 (segment (start 154.32 116.8) (end 157.42 119.9) (width 0.15) (layer F.Cu) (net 9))
 (segment (start 151.405 116.8) (end 151.405 117.275) (width 0.1) (layer F.Cu) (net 9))
 (segment (start 149.25 103.1) (end 147.7 103.1) (width 0.15) (layer F.Cu) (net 10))
 (segment (start 147.7 103.1) (end 146 104.8) (width 0.15) (layer F.Cu) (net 10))
 (segment (start 146 104.8) (end 146 117.64) (width 0.15) (layer F.Cu) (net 10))
 (segment (start 147.26 118.9) (end 147.26 119.9) (width 0.15) (layer F.Cu) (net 10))
 (segment (start 146 117.64) (end 147.26 118.9) (width 0.15) (layer F.Cu) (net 10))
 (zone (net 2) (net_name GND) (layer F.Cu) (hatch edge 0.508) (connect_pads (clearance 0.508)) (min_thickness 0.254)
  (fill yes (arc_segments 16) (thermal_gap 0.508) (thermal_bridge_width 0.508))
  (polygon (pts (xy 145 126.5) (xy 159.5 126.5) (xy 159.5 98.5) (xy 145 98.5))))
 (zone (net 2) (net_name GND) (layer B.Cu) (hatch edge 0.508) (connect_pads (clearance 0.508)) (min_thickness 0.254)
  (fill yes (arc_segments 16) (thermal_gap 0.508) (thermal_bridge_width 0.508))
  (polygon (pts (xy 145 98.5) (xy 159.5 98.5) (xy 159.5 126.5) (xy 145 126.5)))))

